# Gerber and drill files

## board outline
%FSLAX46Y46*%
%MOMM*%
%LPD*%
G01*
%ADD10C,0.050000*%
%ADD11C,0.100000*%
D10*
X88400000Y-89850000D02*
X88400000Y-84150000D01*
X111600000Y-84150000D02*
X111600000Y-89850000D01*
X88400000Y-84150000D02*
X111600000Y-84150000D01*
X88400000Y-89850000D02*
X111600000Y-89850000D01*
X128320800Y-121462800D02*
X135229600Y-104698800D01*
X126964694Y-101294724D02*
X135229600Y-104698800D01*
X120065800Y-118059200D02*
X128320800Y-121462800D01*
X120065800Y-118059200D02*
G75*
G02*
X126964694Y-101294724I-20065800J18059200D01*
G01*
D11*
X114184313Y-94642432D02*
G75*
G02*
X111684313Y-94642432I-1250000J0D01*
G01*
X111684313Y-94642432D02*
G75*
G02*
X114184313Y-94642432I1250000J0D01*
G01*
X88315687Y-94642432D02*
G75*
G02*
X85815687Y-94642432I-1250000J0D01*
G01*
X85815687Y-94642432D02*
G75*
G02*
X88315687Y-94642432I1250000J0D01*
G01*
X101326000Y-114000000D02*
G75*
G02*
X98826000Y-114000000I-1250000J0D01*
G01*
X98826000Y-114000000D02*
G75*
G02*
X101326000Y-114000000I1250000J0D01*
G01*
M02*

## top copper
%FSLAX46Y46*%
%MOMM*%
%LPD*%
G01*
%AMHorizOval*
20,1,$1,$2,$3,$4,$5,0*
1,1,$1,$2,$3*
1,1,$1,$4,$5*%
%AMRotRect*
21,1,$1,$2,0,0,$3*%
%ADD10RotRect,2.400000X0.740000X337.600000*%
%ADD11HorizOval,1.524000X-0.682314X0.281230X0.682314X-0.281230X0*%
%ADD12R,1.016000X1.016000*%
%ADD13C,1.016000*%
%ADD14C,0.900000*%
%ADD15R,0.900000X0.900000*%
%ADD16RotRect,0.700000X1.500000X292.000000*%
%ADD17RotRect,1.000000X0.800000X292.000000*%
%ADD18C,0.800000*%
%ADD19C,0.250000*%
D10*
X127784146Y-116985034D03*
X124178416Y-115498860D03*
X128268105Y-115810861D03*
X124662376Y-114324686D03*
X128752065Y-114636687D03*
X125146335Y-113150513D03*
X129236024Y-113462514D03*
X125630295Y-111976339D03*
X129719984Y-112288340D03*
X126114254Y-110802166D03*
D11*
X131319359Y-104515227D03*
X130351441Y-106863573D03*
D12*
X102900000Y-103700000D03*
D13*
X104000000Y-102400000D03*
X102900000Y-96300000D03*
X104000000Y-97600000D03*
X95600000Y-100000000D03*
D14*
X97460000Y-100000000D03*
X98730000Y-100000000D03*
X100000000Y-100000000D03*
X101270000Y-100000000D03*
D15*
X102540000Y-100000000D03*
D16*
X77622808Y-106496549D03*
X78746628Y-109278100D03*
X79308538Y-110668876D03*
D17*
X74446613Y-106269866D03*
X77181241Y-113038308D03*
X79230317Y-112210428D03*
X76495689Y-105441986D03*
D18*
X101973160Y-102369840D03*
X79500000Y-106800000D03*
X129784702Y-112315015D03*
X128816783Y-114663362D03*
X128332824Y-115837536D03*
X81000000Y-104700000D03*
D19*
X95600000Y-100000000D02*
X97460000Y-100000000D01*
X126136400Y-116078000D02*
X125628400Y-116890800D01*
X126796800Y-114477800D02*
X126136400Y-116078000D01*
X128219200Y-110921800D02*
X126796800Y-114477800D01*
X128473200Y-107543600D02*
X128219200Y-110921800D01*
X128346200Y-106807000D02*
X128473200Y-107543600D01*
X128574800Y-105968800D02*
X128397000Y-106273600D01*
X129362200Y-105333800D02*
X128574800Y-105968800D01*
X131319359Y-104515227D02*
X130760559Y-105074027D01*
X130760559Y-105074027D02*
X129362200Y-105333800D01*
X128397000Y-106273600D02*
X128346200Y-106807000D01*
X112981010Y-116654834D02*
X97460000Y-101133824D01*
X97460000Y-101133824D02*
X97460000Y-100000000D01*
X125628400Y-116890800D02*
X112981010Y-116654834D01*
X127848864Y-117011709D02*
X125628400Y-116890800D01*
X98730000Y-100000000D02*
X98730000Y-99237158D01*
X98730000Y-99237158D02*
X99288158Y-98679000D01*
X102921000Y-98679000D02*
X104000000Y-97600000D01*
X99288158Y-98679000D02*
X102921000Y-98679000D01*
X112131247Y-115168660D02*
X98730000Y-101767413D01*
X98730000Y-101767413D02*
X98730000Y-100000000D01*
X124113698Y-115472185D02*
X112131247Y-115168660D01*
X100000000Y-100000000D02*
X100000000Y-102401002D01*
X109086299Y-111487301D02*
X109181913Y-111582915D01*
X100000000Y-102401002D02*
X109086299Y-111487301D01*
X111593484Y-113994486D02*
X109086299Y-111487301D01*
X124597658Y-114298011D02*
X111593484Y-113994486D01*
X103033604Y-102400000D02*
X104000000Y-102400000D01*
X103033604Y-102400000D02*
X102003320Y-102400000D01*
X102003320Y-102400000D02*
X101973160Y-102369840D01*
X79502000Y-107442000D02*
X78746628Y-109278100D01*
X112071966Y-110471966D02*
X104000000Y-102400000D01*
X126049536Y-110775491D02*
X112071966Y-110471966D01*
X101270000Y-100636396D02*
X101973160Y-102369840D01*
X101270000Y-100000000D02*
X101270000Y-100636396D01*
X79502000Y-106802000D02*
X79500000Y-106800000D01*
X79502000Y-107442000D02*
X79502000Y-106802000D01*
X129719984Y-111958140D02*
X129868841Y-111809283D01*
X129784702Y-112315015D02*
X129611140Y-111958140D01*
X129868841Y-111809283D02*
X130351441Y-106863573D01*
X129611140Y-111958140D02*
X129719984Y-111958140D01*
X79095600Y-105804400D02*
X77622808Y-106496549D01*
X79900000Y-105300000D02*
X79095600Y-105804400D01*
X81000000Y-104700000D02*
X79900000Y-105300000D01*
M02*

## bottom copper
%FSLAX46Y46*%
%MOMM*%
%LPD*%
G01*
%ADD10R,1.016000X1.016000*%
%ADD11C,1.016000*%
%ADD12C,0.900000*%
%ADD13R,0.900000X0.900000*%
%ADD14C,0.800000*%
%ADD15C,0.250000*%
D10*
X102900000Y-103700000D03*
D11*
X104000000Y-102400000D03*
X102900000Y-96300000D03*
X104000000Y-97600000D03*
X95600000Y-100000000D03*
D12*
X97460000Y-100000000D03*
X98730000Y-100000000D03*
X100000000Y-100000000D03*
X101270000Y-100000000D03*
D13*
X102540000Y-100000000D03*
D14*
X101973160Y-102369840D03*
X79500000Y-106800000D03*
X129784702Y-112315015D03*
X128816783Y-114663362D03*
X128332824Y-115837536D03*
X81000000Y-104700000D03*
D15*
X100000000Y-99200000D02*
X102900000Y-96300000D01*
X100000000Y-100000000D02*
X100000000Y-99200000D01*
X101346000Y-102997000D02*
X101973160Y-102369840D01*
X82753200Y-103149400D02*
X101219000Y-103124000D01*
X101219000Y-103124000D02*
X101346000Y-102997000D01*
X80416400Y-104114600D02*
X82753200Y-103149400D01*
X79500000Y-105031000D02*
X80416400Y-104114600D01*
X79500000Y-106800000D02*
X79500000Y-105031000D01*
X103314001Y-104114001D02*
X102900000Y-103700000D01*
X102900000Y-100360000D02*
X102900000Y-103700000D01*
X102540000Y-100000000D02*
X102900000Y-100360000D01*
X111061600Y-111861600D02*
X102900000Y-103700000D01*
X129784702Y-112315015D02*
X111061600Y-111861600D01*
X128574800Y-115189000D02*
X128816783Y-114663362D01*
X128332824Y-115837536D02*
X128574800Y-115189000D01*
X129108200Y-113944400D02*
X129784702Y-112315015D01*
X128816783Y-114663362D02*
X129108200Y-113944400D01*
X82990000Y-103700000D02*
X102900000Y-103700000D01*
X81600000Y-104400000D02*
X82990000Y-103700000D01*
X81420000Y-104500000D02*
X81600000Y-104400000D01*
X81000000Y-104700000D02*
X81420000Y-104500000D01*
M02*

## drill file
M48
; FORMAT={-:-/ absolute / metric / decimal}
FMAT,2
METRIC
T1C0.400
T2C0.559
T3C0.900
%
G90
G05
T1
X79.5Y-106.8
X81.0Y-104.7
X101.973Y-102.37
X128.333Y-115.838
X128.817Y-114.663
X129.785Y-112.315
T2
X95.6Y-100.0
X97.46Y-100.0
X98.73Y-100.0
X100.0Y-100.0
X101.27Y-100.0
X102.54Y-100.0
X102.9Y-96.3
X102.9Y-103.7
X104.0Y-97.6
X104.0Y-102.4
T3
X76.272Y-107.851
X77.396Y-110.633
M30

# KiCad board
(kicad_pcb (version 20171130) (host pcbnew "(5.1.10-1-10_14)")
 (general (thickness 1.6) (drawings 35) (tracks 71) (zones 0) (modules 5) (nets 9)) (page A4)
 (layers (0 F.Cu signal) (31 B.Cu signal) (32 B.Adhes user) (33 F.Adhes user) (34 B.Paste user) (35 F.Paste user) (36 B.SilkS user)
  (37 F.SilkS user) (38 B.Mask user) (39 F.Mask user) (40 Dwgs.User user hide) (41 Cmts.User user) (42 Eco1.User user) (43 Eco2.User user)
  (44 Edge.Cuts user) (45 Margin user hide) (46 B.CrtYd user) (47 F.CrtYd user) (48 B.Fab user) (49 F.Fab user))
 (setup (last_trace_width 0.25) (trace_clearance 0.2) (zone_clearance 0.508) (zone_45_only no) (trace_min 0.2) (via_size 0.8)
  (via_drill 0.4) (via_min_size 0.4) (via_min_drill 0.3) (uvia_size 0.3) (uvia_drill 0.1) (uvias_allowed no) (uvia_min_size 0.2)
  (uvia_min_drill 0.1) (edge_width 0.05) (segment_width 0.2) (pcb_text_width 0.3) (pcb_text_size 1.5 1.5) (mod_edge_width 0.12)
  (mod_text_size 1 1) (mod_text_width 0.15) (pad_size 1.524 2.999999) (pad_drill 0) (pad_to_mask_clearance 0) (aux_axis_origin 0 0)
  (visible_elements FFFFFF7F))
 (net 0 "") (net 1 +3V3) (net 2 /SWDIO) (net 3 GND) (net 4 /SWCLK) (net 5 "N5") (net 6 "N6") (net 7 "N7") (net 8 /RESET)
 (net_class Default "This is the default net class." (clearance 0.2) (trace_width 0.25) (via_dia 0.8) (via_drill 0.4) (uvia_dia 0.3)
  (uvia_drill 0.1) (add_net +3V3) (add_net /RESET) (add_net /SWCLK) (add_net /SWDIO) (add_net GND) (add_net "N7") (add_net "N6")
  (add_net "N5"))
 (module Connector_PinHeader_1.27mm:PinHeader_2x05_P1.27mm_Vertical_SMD (layer F.Cu) (at 126.9492 113.8936 337.6)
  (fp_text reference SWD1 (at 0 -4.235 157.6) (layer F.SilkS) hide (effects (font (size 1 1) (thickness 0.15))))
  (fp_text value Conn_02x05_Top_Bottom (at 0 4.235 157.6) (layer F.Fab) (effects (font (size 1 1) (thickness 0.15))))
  (pad 10 smd rect (at 1.95 2.54 337.6) (size 2.4 0.74) (layers F.Cu F.Paste F.Mask) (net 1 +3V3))
  (pad 9 smd rect (at -1.95 2.54 337.6) (size 2.4 0.74) (layers F.Cu F.Paste F.Mask) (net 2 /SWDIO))
  (pad 8 smd rect (at 1.95 1.27 337.6) (size 2.4 0.74) (layers F.Cu F.Paste F.Mask) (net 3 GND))
  (pad 7 smd rect (at -1.95 1.27 337.6) (size 2.4 0.74) (layers F.Cu F.Paste F.Mask) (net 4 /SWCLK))
  (pad 6 smd rect (at 1.95 0 337.6) (size 2.4 0.74) (layers F.Cu F.Paste F.Mask) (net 3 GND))
  (pad 5 smd rect (at -1.95 0 337.6) (size 2.4 0.74) (layers F.Cu F.Paste F.Mask) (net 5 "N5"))
  (pad 4 smd rect (at 1.95 -1.27 337.6) (size 2.4 0.74) (layers F.Cu F.Paste F.Mask) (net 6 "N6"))
  (pad 3 smd rect (at -1.95 -1.27 337.6) (size 2.4 0.74) (layers F.Cu F.Paste F.Mask) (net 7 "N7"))
  (pad 2 smd rect (at 1.95 -2.54 337.6) (size 2.4 0.74) (layers F.Cu F.Paste F.Mask) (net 3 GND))
  (pad 1 smd rect (at -1.95 -2.54 337.6) (size 2.4 0.74) (layers F.Cu F.Paste F.Mask) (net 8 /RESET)))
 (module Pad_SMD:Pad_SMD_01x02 (layer F.Cu) (at 130.8354 105.6894 247.6)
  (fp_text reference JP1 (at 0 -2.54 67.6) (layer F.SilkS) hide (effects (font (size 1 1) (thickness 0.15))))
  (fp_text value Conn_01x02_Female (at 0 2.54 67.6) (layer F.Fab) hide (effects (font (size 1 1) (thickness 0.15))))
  (pad 1 smd oval (at -1.27 0 247.6) (size 1.524 2.999999) (layers F.Cu F.Paste F.Mask) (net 1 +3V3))
  (pad 2 smd oval (at 1.27 0 247.6) (size 1.524 2.999999) (layers F.Cu F.Paste F.Mask) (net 3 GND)))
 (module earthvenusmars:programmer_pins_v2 (layer F.Cu) (at 100 100)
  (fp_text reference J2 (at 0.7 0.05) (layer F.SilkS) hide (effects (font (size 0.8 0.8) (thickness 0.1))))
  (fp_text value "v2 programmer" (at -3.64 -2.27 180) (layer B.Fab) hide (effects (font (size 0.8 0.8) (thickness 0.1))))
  (pad 5 thru_hole rect (at 2.9 3.7) (size 1.016 1.016) (drill 0.5588) (layers *.Cu *.Mask) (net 3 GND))
  (pad 4 thru_hole circle (at 4 2.4) (size 1.016 1.016) (drill 0.5588) (layers *.Cu *.Mask) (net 8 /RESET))
  (pad 3 thru_hole circle (at 2.9 -3.7) (size 1.016 1.016) (drill 0.5588) (layers *.Cu *.Mask) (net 4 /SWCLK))
  (pad 2 thru_hole circle (at 4 -2.4) (size 1.016 1.016) (drill 0.5588) (layers *.Cu *.Mask) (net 2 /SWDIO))
  (pad 1 thru_hole circle (at -4.4 0) (size 1.016 1.016) (drill 0.5588) (layers *.Cu *.Mask) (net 1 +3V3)))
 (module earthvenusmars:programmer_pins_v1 (layer F.Cu) (at 100 100)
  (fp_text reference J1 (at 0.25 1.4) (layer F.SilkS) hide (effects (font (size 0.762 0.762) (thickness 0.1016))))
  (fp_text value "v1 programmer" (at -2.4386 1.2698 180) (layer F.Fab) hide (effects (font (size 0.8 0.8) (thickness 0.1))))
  (pad 1 thru_hole circle (at -2.54 0) (size 0.9 0.9) (drill 0.5588) (layers *.Cu *.Mask) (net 1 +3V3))
  (pad 2 thru_hole circle (at -1.27 0) (size 0.9 0.9) (drill 0.5588) (layers *.Cu *.Mask) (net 2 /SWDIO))
  (pad 3 thru_hole circle (at 0 0) (size 0.9 0.9) (drill 0.5588) (layers *.Cu *.Mask) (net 4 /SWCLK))
  (pad 4 thru_hole circle (at 1.27 0) (size 0.9 0.9) (drill 0.5588) (layers *.Cu *.Mask) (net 8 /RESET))
  (pad 5 thru_hole rect (at 2.54 0) (size 0.9 0.9) (drill 0.5588) (layers *.Cu *.Mask) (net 3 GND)))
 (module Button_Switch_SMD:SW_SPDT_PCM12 (layer F.Cu) (at 77.1398 109.1184 292)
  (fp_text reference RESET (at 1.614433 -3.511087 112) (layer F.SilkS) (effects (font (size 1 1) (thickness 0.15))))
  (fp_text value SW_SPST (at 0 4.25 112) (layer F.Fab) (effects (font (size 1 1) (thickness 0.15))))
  (pad "" np_thru_hole circle (at -1.5 0.33 292) (size 0.9 0.9) (drill 0.9) (layers *.Cu *.Mask))
  (pad "" np_thru_hole circle (at 1.5 0.33 292) (size 0.9 0.9) (drill 0.9) (layers *.Cu *.Mask))
  (pad 1 smd rect (at -2.25 -1.43 292) (size 0.7 1.5) (layers F.Cu F.Paste F.Mask) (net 3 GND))
  (pad 2 smd rect (at 0.75 -1.43 292) (size 0.7 1.5) (layers F.Cu F.Paste F.Mask) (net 8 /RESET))
  (pad 3 smd rect (at 2.25 -1.43 292) (size 0.7 1.5) (layers F.Cu F.Paste F.Mask))
  (pad "" smd rect (at -3.65 1.43 292) (size 1 0.8) (layers F.Cu F.Paste F.Mask))
  (pad "" smd rect (at 3.65 1.43 292) (size 1 0.8) (layers F.Cu F.Paste F.Mask))
  (pad "" smd rect (at 3.65 -0.78 292) (size 1 0.8) (layers F.Cu F.Paste F.Mask))
  (pad "" smd rect (at -3.65 -0.78 292) (size 1 0.8) (layers F.Cu F.Paste F.Mask)))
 (gr_line (start 88.4 89.85) (end 88.4 84.15) (layer Edge.Cuts) (width 0.05))
 (gr_line (start 111.6 84.15) (end 111.6 89.85) (layer Edge.Cuts) (width 0.05))
 (gr_line (start 88.4 84.15) (end 111.6 84.15) (layer Edge.Cuts) (width 0.05))
 (gr_line (start 88.4 89.85) (end 111.6 89.85) (layer Edge.Cuts) (width 0.05))
 (gr_line (start 128.3208 121.4628) (end 135.2296 104.6988) (layer Edge.Cuts) (width 0.05))
 (gr_line (start 126.964694 101.294724) (end 135.2296 104.6988) (layer Edge.Cuts) (width 0.05))
 (gr_line (start 120.0658 118.0592) (end 128.3208 121.4628) (layer Edge.Cuts) (width 0.05))
 (gr_arc (start 100 100) (end 120.0658 118.0592) (angle 320.7617956) (layer Edge.Cuts) (width 0.05))
 (gr_circle (center 112.934313 94.642432) (end 114.184313 94.642432) (layer Edge.Cuts) (width 0.1))
 (gr_circle (center 87.065687 94.642432) (end 88.315687 94.642432) (layer Edge.Cuts) (width 0.1))
 (gr_circle (center 100.076 114) (end 101.326 114) (layer Edge.Cuts) (width 0.1))
 (segment (start 95.6 100) (end 97.46 100) (width 0.25) (layer F.Cu) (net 1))
 (segment (start 126.1364 116.078) (end 125.6284 116.8908) (width 0.25) (layer F.Cu) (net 1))
 (segment (start 126.7968 114.4778) (end 126.1364 116.078) (width 0.25) (layer F.Cu) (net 1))
 (segment (start 128.2192 110.9218) (end 126.7968 114.4778) (width 0.25) (layer F.Cu) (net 1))
 (segment (start 128.4732 107.5436) (end 128.2192 110.9218) (width 0.25) (layer F.Cu) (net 1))
 (segment (start 128.3462 106.807) (end 128.4732 107.5436) (width 0.25) (layer F.Cu) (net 1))
 (segment (start 128.5748 105.9688) (end 128.397 106.2736) (width 0.25) (layer F.Cu) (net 1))
 (segment (start 129.3622 105.3338) (end 128.5748 105.9688) (width 0.25) (layer F.Cu) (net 1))
 (segment (start 131.319359 104.515227) (end 130.760559 105.074027) (width 0.25) (layer F.Cu) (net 1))
 (segment (start 130.760559 105.074027) (end 129.3622 105.3338) (width 0.25) (layer F.Cu) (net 1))
 (segment (start 128.397 106.2736) (end 128.3462 106.807) (width 0.25) (layer F.Cu) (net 1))
 (segment (start 112.98101 116.654834) (end 97.46 101.133824) (width 0.25) (layer F.Cu) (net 1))
 (segment (start 97.46 101.133824) (end 97.46 100) (width 0.25) (layer F.Cu) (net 1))
 (segment (start 125.6284 116.8908) (end 112.98101 116.654834) (width 0.25) (layer F.Cu) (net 1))
 (segment (start 127.848864 117.011709) (end 125.6284 116.8908) (width 0.25) (layer F.Cu) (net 1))
 (segment (start 98.73 100) (end 98.73 99.237158) (width 0.25) (layer F.Cu) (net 2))
 (segment (start 98.73 99.237158) (end 99.288158 98.679) (width 0.25) (layer F.Cu) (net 2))
 (segment (start 102.921 98.679) (end 104 97.6) (width 0.25) (layer F.Cu) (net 2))
 (segment (start 99.288158 98.679) (end 102.921 98.679) (width 0.25) (layer F.Cu) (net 2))
 (segment (start 112.131247 115.16866) (end 98.73 101.767413) (width 0.25) (layer F.Cu) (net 2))
 (segment (start 98.73 101.767413) (end 98.73 100) (width 0.25) (layer F.Cu) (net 2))
 (segment (start 124.113698 115.472185) (end 112.131247 115.16866) (width 0.25) (layer F.Cu) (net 2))
 (segment (start 100 100) (end 100 102.401002) (width 0.25) (layer F.Cu) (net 4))
 (segment (start 109.086299 111.487301) (end 109.181913 111.582915) (width 0.25) (layer F.Cu) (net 4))
 (segment (start 100 102.401002) (end 109.086299 111.487301) (width 0.25) (layer F.Cu) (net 4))
 (segment (start 111.593484 113.994486) (end 109.086299 111.487301) (width 0.25) (layer F.Cu) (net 4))
 (segment (start 124.597658 114.298011) (end 111.593484 113.994486) (width 0.25) (layer F.Cu) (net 4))
 (segment (start 100 99.2) (end 102.9 96.3) (width 0.25) (layer B.Cu) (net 4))
 (segment (start 100 100) (end 100 99.2) (width 0.25) (layer B.Cu) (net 4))
 (segment (start 103.033604 102.4) (end 104 102.4) (width 0.25) (layer F.Cu) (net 8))
 (via (at 101.97316 102.36984) (size 0.8) (drill 0.4) (layers F.Cu B.Cu) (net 8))
 (segment (start 103.033604 102.4) (end 102.00332 102.4) (width 0.25) (layer F.Cu) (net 8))
 (segment (start 102.00332 102.4) (end 101.97316 102.36984) (width 0.25) (layer F.Cu) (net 8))
 (segment (start 101.346 102.997) (end 101.97316 102.36984) (width 0.25) (layer B.Cu) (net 8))
 (segment (start 82.7532 103.1494) (end 101.219 103.124) (width 0.25) (layer B.Cu) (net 8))
 (segment (start 101.219 103.124) (end 101.346 102.997) (width 0.25) (layer B.Cu) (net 8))
 (segment (start 80.4164 104.1146) (end 82.7532 103.1494) (width 0.25) (layer B.Cu) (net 8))
 (segment (start 79.502 107.442) (end 78.746628 109.2781) (width 0.25) (layer F.Cu) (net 8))
 (segment (start 112.071966 110.471966) (end 104 102.4) (width 0.25) (layer F.Cu) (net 8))
 (segment (start 126.049536 110.775491) (end 112.071966 110.471966) (width 0.25) (layer F.Cu) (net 8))
 (segment (start 101.27 100.636396) (end 101.97316 102.36984) (width 0.25) (layer F.Cu) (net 8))
 (segment (start 101.27 100) (end 101.27 100.636396) (width 0.25) (layer F.Cu) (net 8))
 (via (at 79.5 106.8) (size 0.8) (drill 0.4) (layers F.Cu B.Cu) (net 8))
 (segment (start 79.502 106.802) (end 79.5 106.8) (width 0.25) (layer F.Cu) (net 8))
 (segment (start 79.502 107.442) (end 79.502 106.802) (width 0.25) (layer F.Cu) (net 8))
 (segment (start 79.5 105.031) (end 80.4164 104.1146) (width 0.25) (layer B.Cu) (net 8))
 (segment (start 79.5 106.8) (end 79.5 105.031) (width 0.25) (layer B.Cu) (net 8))
 (segment (start 103.314001 104.114001) (end 102.9 103.7) (width 0.25) (layer B.Cu) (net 3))
 (segment (start 102.9 100.36) (end 102.9 103.7) (width 0.25) (layer B.Cu) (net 3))
 (segment (start 102.54 100) (end 102.9 100.36) (width 0.25) (layer B.Cu) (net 3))
 (segment (start 129.719984 111.95814) (end 129.868841 111.809283) (width 0.25) (layer F.Cu) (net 3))
 (segment (start 129.784702 112.315015) (end 129.61114 111.95814) (width 0.25) (layer F.Cu) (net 3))
 (segment (start 111.0616 111.8616) (end 102.9 103.7) (width 0.25) (layer B.Cu) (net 3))
 (segment (start 129.784702 112.315015) (end 111.0616 111.8616) (width 0.25) (layer B.Cu) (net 3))
 (segment (start 129.868841 111.809283) (end 130.351441 106.863573) (width 0.25) (layer F.Cu) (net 3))
 (segment (start 129.61114 111.95814) (end 129.719984 111.95814) (width 0.25) (layer F.Cu) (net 3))
 (via (at 129.784702 112.315015) (size 0.8) (drill 0.4) (layers F.Cu B.Cu) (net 3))
 (via (at 128.816783 114.663362) (size 0.8) (drill 0.4) (layers F.Cu B.Cu) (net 3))
 (via (at 128.332824 115.837536) (size 0.8) (drill 0.4) (layers F.Cu B.Cu) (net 3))
 (segment (start 128.5748 115.189) (end 128.816783 114.663362) (width 0.25) (layer B.Cu) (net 3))
 (segment (start 128.332824 115.837536) (end 128.5748 115.189) (width 0.25) (layer B.Cu) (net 3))
 (segment (start 129.1082 113.9444) (end 129.784702 112.315015) (width 0.25) (layer B.Cu) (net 3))
 (segment (start 128.816783 114.663362) (end 129.1082 113.9444) (width 0.25) (layer B.Cu) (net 3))
 (via (at 81 104.7) (size 0.8) (drill 0.4) (layers F.Cu B.Cu) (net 3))
 (segment (start 82.99 103.7) (end 102.9 103.7) (width 0.25) (layer B.Cu) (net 3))
 (segment (start 81.6 104.4) (end 82.99 103.7) (width 0.25) (layer B.Cu) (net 3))
 (segment (start 81.42 104.5) (end 81.6 104.4) (width 0.25) (layer B.Cu) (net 3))
 (segment (start 81 104.7) (end 81.42 104.5) (width 0.25) (layer B.Cu) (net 3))
 (segment (start 79.0956 105.8044) (end 77.622808 106.496549) (width 0.25) (layer F.Cu) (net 3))
 (segment (start 79.9 105.3) (end 79.0956 105.8044) (width 0.25) (layer F.Cu) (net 3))
 (segment (start 81 104.7) (end 79.9 105.3) (width 0.25) (layer F.Cu) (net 3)))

